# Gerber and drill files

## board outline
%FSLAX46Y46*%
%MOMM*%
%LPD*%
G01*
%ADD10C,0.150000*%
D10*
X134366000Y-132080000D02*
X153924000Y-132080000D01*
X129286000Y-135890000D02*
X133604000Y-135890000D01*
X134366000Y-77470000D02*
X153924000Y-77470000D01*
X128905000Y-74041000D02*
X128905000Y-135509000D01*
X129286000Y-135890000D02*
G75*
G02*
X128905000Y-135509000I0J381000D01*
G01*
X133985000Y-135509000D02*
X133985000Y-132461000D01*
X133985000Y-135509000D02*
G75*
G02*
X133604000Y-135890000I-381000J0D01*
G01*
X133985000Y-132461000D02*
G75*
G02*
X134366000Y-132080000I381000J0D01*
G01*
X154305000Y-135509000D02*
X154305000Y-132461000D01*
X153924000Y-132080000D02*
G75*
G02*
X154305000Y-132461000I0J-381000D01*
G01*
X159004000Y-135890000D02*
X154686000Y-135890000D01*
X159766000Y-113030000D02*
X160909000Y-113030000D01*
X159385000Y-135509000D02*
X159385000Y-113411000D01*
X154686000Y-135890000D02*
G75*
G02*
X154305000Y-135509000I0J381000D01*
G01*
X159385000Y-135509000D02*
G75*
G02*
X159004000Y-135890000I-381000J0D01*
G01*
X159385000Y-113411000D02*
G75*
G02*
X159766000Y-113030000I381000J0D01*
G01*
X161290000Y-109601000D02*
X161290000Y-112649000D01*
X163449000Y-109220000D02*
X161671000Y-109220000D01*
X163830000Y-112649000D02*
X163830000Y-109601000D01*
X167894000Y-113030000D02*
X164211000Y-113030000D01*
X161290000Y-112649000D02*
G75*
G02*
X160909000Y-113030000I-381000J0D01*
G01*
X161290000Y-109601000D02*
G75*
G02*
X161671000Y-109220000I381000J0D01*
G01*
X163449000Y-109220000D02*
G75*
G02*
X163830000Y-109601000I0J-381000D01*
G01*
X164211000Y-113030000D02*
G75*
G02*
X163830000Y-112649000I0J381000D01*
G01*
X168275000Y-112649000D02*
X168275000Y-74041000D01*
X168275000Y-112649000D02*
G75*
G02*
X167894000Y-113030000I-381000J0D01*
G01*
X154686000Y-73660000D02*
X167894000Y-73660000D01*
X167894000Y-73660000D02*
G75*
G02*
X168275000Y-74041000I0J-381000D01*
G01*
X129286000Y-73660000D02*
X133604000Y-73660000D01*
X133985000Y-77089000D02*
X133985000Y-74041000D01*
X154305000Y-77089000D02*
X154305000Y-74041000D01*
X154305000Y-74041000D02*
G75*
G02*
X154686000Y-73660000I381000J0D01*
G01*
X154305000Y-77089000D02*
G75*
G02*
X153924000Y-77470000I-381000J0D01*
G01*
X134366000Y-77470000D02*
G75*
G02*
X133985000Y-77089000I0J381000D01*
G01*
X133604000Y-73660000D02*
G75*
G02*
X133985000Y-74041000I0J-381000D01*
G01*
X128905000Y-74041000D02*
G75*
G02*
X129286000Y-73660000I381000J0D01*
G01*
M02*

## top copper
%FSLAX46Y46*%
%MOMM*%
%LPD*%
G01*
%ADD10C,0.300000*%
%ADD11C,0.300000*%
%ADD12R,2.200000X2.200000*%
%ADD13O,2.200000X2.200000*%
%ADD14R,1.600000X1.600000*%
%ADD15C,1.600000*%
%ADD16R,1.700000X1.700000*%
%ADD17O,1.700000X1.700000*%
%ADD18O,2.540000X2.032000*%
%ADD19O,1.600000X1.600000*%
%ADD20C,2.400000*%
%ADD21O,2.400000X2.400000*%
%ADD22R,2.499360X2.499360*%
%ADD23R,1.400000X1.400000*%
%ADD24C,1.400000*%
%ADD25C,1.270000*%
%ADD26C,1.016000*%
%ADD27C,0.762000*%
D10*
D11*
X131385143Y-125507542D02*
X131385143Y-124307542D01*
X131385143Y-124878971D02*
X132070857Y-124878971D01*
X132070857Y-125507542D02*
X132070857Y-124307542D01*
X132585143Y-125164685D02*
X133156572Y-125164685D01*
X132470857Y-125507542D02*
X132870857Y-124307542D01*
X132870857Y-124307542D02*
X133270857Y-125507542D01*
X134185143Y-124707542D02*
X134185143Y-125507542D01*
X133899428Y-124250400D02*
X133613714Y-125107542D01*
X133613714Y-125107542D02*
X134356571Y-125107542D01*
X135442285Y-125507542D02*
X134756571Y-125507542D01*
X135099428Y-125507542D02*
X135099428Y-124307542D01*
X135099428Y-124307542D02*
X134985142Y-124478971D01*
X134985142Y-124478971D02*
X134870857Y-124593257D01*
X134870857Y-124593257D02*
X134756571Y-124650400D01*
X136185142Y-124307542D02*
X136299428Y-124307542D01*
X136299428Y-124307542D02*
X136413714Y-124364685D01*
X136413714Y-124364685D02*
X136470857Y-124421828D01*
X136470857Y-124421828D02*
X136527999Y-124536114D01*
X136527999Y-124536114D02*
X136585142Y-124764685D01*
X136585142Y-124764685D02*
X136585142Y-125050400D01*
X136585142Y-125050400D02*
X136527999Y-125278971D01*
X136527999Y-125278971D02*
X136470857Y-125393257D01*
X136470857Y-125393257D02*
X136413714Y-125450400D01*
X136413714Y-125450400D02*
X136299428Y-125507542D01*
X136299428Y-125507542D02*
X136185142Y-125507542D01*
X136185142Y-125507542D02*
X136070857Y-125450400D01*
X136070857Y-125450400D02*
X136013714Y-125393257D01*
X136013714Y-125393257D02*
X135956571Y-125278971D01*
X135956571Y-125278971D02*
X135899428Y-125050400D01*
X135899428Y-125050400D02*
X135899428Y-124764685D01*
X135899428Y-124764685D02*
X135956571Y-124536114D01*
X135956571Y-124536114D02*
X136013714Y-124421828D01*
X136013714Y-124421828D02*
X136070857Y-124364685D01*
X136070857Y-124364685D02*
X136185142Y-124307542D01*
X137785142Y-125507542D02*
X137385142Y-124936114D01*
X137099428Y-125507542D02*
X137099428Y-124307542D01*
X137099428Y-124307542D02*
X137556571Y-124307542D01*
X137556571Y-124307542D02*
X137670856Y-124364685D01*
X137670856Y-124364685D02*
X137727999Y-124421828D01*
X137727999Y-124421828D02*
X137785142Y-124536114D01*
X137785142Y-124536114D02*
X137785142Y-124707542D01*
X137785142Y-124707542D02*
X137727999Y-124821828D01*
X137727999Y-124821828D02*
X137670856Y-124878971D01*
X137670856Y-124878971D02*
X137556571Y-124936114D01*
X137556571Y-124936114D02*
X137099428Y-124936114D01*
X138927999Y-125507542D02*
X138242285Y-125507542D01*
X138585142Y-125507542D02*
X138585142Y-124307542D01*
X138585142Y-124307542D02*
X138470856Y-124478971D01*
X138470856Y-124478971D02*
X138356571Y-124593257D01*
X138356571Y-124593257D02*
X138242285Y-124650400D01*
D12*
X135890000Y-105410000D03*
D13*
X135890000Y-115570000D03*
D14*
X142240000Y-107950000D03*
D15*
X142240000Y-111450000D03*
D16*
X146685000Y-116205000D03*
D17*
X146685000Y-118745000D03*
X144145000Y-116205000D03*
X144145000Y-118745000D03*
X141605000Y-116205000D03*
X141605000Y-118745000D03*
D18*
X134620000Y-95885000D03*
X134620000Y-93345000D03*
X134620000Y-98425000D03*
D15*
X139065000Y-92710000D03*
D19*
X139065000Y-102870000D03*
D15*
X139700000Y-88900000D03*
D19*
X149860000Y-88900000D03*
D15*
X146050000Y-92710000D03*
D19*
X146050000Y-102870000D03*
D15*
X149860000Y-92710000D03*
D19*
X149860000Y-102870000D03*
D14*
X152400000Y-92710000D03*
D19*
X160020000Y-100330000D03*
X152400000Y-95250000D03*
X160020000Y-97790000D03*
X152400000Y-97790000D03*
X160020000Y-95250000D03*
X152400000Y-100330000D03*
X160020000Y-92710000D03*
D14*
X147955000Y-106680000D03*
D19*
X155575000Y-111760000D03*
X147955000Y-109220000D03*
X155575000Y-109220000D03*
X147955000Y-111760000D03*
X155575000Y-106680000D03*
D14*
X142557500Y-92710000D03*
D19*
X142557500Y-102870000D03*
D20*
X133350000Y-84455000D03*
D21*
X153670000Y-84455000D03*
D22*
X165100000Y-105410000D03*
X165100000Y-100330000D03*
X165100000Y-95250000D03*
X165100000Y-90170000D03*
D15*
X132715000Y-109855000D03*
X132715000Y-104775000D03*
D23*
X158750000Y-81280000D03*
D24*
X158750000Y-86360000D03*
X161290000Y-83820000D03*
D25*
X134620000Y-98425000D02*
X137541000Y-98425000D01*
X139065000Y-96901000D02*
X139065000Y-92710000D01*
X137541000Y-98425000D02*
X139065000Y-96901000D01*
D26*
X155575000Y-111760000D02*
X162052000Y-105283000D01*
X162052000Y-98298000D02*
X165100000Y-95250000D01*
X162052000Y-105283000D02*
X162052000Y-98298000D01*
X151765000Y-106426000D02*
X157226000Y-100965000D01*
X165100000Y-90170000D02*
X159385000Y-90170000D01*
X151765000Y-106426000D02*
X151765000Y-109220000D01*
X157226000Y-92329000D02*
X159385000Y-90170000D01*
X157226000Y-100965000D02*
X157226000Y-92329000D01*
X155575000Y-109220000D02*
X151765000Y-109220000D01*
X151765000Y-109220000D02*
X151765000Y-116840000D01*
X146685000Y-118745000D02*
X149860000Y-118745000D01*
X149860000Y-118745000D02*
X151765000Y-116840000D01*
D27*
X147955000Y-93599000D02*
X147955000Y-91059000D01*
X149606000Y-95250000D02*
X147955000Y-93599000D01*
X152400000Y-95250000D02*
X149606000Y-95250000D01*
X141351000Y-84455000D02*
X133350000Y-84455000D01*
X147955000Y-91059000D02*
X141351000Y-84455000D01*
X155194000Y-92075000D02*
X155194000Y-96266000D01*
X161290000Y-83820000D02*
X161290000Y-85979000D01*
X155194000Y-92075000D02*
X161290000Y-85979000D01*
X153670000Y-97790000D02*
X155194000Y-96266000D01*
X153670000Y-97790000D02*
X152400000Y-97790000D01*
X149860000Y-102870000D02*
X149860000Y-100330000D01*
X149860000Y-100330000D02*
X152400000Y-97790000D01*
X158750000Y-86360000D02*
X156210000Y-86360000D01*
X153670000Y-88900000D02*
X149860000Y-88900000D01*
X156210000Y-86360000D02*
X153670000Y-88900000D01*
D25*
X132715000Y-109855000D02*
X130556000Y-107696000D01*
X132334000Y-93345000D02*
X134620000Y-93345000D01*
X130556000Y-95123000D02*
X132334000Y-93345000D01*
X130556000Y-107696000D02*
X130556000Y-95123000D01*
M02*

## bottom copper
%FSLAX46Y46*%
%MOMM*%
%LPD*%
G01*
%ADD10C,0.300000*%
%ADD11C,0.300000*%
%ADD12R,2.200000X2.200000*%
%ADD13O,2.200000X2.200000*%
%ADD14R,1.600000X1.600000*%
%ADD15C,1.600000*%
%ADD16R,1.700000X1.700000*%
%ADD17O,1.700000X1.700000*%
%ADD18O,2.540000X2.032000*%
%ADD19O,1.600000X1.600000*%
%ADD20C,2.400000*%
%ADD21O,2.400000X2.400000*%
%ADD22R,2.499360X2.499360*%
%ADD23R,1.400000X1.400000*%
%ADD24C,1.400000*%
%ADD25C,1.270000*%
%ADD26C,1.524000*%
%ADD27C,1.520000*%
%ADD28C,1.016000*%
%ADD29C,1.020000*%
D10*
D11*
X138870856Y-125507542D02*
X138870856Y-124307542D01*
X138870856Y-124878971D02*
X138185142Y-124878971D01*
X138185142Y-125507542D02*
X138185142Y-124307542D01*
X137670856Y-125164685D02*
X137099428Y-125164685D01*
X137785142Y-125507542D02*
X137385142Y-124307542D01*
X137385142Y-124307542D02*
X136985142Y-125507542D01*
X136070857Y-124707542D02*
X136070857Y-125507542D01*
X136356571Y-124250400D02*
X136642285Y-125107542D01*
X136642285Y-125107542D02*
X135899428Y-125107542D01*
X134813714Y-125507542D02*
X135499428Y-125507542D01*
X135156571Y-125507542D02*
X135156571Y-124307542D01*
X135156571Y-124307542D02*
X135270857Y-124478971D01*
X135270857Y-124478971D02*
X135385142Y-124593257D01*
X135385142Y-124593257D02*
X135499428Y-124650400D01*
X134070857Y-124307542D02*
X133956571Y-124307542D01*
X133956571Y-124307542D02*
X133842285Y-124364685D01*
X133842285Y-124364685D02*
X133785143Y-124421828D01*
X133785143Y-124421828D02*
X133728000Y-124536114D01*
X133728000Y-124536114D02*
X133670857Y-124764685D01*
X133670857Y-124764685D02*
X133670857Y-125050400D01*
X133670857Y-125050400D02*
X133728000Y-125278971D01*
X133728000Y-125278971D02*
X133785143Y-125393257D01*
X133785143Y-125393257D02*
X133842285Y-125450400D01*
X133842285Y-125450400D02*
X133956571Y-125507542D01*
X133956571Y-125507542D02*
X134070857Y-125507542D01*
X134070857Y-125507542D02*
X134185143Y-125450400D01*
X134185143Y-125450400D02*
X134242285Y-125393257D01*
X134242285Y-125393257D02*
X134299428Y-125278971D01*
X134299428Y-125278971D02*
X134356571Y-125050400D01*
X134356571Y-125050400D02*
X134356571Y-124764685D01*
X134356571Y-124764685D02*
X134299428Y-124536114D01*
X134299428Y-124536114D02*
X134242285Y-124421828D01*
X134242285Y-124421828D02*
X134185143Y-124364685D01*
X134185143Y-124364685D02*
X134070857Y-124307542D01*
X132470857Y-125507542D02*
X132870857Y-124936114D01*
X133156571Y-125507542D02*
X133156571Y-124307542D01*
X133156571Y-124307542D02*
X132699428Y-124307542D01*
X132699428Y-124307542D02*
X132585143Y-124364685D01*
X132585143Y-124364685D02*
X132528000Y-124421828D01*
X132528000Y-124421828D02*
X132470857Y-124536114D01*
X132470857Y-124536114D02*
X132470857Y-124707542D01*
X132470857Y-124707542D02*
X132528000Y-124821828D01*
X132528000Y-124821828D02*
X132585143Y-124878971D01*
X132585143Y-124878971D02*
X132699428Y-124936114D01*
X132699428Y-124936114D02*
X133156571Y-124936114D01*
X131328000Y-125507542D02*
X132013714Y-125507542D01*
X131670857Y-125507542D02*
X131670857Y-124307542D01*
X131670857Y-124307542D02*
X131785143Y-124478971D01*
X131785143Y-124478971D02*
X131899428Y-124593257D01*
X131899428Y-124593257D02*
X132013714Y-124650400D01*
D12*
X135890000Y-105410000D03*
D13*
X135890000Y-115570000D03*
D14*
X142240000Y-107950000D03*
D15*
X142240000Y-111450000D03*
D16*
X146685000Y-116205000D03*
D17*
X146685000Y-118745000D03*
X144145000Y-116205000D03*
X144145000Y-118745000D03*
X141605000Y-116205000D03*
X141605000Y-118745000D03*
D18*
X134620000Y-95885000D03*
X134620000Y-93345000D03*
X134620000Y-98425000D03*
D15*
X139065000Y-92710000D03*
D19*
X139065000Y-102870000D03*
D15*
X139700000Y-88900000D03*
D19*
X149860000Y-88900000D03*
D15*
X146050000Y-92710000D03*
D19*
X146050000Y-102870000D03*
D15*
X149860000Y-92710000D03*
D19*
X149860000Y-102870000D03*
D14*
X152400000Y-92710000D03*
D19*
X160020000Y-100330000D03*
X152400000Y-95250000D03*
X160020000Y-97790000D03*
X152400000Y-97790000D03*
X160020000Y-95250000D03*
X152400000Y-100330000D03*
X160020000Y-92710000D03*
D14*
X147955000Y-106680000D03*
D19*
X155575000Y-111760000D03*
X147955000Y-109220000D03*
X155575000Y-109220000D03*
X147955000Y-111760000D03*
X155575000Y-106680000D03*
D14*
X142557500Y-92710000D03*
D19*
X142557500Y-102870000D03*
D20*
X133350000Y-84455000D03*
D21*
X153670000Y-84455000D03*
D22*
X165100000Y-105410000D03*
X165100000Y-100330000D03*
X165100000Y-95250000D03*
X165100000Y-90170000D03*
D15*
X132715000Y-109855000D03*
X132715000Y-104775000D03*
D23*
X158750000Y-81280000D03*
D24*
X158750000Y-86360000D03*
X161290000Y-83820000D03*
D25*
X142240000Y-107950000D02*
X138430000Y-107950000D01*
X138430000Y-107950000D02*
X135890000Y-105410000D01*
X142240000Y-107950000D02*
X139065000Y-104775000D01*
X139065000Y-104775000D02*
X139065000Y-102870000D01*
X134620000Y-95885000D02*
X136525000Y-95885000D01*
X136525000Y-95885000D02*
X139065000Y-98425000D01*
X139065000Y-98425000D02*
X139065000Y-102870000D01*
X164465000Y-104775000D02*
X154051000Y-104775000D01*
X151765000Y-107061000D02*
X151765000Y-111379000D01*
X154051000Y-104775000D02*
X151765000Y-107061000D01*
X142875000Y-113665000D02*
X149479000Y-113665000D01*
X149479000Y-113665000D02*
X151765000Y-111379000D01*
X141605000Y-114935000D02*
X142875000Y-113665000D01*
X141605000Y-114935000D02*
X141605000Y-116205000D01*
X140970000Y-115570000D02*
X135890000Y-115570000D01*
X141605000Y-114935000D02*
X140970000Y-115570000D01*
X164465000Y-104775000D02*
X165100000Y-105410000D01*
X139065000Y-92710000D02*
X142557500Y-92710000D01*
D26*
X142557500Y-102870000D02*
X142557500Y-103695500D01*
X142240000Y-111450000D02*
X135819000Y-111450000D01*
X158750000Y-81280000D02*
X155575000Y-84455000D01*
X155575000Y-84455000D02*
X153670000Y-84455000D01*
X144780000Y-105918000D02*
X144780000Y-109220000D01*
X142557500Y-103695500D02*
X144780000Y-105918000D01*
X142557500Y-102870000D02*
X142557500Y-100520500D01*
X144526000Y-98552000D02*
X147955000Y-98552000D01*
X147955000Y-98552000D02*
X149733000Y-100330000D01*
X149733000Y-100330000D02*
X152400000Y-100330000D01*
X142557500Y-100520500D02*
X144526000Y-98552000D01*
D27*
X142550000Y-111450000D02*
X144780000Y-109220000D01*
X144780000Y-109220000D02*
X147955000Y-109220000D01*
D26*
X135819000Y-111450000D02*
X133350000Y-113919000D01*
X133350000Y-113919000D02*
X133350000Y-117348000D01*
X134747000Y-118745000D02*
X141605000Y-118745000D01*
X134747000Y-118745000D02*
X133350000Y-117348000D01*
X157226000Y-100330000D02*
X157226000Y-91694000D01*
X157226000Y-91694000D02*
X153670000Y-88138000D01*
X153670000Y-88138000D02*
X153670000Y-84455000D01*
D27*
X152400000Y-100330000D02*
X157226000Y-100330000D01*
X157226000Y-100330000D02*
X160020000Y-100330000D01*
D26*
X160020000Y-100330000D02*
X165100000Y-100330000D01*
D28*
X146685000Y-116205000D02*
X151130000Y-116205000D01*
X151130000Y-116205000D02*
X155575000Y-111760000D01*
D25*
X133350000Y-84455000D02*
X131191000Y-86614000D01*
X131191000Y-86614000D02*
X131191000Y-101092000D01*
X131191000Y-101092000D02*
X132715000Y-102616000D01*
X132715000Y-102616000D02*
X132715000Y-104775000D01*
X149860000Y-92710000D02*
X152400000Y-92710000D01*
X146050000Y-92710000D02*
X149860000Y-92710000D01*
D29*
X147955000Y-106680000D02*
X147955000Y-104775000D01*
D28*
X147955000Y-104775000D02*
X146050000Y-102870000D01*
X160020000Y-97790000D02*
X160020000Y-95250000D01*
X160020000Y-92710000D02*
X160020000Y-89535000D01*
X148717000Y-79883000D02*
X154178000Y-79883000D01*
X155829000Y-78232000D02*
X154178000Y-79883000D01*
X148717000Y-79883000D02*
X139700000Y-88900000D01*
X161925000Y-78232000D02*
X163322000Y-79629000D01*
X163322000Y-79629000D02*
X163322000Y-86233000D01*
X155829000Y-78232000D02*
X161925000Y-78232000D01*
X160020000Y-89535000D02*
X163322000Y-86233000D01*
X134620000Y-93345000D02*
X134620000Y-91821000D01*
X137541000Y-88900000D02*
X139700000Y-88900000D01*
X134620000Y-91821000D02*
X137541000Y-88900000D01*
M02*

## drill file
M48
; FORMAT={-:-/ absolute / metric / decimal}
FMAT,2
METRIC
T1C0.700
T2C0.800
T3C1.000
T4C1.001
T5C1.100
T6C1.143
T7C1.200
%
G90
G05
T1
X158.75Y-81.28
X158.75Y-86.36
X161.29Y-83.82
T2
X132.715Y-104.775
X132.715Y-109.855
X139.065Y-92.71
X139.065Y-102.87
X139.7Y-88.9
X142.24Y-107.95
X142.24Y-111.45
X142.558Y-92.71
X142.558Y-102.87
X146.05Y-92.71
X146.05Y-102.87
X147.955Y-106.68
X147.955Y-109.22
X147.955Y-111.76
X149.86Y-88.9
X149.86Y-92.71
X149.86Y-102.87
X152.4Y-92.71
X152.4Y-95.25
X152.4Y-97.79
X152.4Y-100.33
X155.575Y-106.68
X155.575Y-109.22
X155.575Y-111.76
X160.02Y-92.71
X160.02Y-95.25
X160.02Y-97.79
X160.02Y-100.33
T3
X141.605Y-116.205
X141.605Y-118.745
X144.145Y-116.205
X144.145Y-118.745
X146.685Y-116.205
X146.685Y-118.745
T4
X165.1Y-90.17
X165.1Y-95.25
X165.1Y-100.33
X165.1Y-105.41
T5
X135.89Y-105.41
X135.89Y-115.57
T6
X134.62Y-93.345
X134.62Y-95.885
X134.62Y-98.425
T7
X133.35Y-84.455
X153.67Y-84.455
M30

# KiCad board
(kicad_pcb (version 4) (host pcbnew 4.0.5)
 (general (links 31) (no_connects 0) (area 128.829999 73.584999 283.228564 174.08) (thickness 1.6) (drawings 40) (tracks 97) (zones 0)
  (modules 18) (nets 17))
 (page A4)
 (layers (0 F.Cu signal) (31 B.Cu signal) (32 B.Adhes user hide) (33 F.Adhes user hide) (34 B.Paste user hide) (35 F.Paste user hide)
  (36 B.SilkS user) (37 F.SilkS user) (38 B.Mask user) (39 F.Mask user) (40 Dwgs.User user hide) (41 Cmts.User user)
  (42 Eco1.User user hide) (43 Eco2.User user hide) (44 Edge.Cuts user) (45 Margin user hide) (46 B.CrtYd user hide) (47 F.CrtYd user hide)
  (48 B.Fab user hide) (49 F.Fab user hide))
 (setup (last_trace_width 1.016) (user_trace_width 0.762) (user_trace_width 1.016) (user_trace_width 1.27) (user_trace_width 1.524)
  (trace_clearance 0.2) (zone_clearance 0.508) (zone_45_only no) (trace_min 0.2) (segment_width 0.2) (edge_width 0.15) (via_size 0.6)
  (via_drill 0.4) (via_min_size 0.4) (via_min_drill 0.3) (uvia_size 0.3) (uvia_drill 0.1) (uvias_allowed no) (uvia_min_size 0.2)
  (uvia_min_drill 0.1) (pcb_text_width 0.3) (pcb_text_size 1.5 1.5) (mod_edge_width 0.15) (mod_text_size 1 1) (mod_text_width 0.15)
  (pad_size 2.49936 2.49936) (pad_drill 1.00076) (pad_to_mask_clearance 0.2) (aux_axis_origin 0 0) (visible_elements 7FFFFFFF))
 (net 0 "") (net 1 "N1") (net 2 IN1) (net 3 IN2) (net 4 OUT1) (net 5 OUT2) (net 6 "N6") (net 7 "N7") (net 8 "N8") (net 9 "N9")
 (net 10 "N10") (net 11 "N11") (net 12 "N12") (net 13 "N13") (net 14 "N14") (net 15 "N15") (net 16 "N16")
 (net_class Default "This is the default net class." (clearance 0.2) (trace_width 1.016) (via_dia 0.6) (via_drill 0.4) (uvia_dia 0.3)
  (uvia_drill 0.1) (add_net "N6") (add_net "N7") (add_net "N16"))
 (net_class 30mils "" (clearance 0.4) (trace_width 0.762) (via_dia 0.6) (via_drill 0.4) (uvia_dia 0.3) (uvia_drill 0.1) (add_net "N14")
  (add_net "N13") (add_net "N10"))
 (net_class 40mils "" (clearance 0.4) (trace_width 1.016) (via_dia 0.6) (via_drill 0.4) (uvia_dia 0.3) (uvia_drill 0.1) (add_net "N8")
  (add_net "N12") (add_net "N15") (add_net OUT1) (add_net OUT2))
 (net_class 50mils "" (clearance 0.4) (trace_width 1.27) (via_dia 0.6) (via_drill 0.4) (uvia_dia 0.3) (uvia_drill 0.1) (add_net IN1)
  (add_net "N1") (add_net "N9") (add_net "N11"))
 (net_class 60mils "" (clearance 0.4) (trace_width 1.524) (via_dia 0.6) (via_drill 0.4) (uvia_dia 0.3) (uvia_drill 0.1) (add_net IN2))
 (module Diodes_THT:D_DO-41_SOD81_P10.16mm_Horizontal (layer F.Cu) (at 135.89 105.41 270)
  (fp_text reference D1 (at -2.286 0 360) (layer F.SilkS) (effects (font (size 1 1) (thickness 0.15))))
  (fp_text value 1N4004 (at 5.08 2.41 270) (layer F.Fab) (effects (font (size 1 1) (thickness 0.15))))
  (pad 1 thru_hole rect (at 0 0 270) (size 2.2 2.2) (drill 1.1) (layers *.Cu *.Mask) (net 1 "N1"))
  (pad 2 thru_hole oval (at 10.16 0 270) (size 2.2 2.2) (drill 1.1) (layers *.Cu *.Mask) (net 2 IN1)))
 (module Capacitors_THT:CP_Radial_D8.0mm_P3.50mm (layer F.Cu) (at 142.24 107.95 270)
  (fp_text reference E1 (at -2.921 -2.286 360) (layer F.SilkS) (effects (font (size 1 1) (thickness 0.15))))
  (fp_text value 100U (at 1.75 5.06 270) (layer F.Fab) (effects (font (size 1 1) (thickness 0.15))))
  (pad 1 thru_hole rect (at 0 0 270) (size 1.6 1.6) (drill 0.8) (layers *.Cu *.Mask) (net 1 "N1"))
  (pad 2 thru_hole circle (at 3.5 0 270) (size 1.6 1.6) (drill 0.8) (layers *.Cu *.Mask) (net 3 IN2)))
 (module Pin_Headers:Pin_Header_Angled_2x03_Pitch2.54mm (layer F.Cu) (at 146.685 116.205 270)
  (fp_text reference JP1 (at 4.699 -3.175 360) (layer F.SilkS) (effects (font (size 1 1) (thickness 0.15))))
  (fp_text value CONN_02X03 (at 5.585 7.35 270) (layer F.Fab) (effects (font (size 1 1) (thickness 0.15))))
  (pad 1 thru_hole rect (at 0 0 270) (size 1.7 1.7) (drill 1) (layers *.Cu *.Mask) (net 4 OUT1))
  (pad 2 thru_hole oval (at 2.54 0 270) (size 1.7 1.7) (drill 1) (layers *.Cu *.Mask) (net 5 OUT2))
  (pad 3 thru_hole oval (at 0 2.54 270) (size 1.7 1.7) (drill 1) (layers *.Cu *.Mask) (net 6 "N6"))
  (pad 4 thru_hole oval (at 2.54 2.54 270) (size 1.7 1.7) (drill 1) (layers *.Cu *.Mask) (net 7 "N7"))
  (pad 5 thru_hole oval (at 0 5.08 270) (size 1.7 1.7) (drill 1) (layers *.Cu *.Mask) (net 2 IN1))
  (pad 6 thru_hole oval (at 2.54 5.08 270) (size 1.7 1.7) (drill 1) (layers *.Cu *.Mask) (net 3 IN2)))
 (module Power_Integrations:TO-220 (layer F.Cu) (at 134.62 95.885 90)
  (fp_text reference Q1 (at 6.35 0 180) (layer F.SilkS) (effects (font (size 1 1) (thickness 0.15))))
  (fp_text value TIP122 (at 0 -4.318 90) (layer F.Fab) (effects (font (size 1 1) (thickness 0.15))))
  (pad 2 thru_hole oval (at 0 0 90) (size 2.032 2.54) (drill 1.143) (layers *.Cu *.Mask) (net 1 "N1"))
  (pad 3 thru_hole oval (at 2.54 0 90) (size 2.032 2.54) (drill 1.143) (layers *.Cu *.Mask) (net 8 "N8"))
  (pad 1 thru_hole oval (at -2.54 0 90) (size 2.032 2.54) (drill 1.143) (layers *.Cu *.Mask) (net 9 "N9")))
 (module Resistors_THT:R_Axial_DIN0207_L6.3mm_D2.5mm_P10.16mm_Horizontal (layer F.Cu) (at 139.065 92.71 270)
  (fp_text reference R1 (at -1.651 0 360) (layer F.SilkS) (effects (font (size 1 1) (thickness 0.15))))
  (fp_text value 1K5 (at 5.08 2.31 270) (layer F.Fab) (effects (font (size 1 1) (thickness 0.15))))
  (pad 1 thru_hole circle (at 0 0 270) (size 1.6 1.6) (drill 0.8) (layers *.Cu *.Mask) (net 9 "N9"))
  (pad 2 thru_hole oval (at 10.16 0 270) (size 1.6 1.6) (drill 0.8) (layers *.Cu *.Mask) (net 1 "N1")))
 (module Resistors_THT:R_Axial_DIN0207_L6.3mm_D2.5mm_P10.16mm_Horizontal (layer F.Cu) (at 139.7 88.9)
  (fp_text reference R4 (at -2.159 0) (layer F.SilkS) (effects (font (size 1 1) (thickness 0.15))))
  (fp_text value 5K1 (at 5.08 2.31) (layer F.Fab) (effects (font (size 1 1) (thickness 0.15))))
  (pad 1 thru_hole circle (at 0 0) (size 1.6 1.6) (drill 0.8) (layers *.Cu *.Mask) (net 8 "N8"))
  (pad 2 thru_hole oval (at 10.16 0) (size 1.6 1.6) (drill 0.8) (layers *.Cu *.Mask) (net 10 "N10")))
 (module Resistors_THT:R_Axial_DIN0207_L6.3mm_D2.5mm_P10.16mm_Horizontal (layer F.Cu) (at 146.05 92.71 270)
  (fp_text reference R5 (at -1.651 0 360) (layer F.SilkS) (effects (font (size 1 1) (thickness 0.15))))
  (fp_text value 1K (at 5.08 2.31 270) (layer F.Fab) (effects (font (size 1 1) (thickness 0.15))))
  (pad 1 thru_hole circle (at 0 0 270) (size 1.6 1.6) (drill 0.8) (layers *.Cu *.Mask) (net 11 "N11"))
  (pad 2 thru_hole oval (at 10.16 0 270) (size 1.6 1.6) (drill 0.8) (layers *.Cu *.Mask) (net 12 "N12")))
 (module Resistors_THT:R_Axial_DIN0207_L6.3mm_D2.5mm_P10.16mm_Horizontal (layer F.Cu) (at 149.86 92.71 270)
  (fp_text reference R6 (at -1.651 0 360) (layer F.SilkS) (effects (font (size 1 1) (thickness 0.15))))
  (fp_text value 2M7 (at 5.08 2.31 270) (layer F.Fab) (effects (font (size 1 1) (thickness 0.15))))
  (pad 1 thru_hole circle (at 0 0 270) (size 1.6 1.6) (drill 0.8) (layers *.Cu *.Mask) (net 11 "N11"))
  (pad 2 thru_hole oval (at 10.16 0 270) (size 1.6 1.6) (drill 0.8) (layers *.Cu *.Mask) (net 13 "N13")))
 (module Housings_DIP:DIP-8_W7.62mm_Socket (layer F.Cu) (at 152.4 92.71)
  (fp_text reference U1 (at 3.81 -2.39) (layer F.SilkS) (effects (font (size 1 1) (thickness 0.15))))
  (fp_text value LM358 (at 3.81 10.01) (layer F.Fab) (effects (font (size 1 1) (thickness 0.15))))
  (pad 1 thru_hole rect (at 0 0) (size 1.6 1.6) (drill 0.8) (layers *.Cu *.Mask) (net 11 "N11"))
  (pad 5 thru_hole oval (at 7.62 7.62) (size 1.6 1.6) (drill 0.8) (layers *.Cu *.Mask) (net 3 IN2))
  (pad 2 thru_hole oval (at 0 2.54) (size 1.6 1.6) (drill 0.8) (layers *.Cu *.Mask) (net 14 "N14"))
  (pad 6 thru_hole oval (at 7.62 5.08) (size 1.6 1.6) (drill 0.8) (layers *.Cu *.Mask) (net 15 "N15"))
  (pad 3 thru_hole oval (at 0 5.08) (size 1.6 1.6) (drill 0.8) (layers *.Cu *.Mask) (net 13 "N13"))
  (pad 7 thru_hole oval (at 7.62 2.54) (size 1.6 1.6) (drill 0.8) (layers *.Cu *.Mask) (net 15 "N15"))
  (pad 4 thru_hole oval (at 0 7.62) (size 1.6 1.6) (drill 0.8) (layers *.Cu *.Mask) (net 3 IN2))
  (pad 8 thru_hole oval (at 7.62 0) (size 1.6 1.6) (drill 0.8) (layers *.Cu *.Mask) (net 8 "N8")))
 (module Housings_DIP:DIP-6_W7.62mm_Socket (layer F.Cu) (at 147.955 106.68)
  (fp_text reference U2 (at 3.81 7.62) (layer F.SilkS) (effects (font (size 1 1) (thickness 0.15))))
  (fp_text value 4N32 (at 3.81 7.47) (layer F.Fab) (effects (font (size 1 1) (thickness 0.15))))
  (pad 1 thru_hole rect (at 0 0) (size 1.6 1.6) (drill 0.8) (layers *.Cu *.Mask) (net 12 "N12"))
  (pad 4 thru_hole oval (at 7.62 5.08) (size 1.6 1.6) (drill 0.8) (layers *.Cu *.Mask) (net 4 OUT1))
  (pad 2 thru_hole oval (at 0 2.54) (size 1.6 1.6) (drill 0.8) (layers *.Cu *.Mask) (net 3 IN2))
  (pad 5 thru_hole oval (at 7.62 2.54) (size 1.6 1.6) (drill 0.8) (layers *.Cu *.Mask) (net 5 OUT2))
  (pad 3 thru_hole oval (at 0 5.08) (size 1.6 1.6) (drill 0.8) (layers *.Cu *.Mask))
  (pad 6 thru_hole oval (at 7.62 0) (size 1.6 1.6) (drill 0.8) (layers *.Cu *.Mask) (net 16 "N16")))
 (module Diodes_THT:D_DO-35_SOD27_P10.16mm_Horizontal (layer F.Cu) (at 142.5575 92.71 270)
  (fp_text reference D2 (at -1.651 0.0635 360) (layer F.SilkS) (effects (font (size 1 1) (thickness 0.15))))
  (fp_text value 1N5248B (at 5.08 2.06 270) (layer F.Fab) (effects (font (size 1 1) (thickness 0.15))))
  (pad 1 thru_hole rect (at 0 0 270) (size 1.6 1.6) (drill 0.8) (layers *.Cu *.Mask) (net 9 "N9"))
  (pad 2 thru_hole oval (at 10.16 0 270) (size 1.6 1.6) (drill 0.8) (layers *.Cu *.Mask) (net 3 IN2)))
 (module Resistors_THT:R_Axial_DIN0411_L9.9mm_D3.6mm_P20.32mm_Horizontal (layer F.Cu) (at 133.35 84.455)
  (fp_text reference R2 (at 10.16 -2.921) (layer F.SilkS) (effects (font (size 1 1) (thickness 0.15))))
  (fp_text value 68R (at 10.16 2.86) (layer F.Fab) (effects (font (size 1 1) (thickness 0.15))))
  (pad 1 thru_hole circle (at 0 0) (size 2.4 2.4) (drill 1.2) (layers *.Cu *.Mask) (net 14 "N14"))
  (pad 2 thru_hole oval (at 20.32 0) (size 2.4 2.4) (drill 1.2) (layers *.Cu *.Mask) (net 3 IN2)))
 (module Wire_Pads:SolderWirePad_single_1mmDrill (layer F.Cu) (at 165.1 105.41)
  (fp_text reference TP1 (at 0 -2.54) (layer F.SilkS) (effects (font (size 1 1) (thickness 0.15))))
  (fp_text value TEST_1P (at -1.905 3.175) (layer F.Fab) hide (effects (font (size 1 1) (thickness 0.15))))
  (pad 1 thru_hole rect (at 0 0) (size 2.49936 2.49936) (drill 1.00076) (layers *.Cu *.Mask) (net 2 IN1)))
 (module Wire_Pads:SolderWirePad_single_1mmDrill (layer F.Cu) (at 165.1 100.33)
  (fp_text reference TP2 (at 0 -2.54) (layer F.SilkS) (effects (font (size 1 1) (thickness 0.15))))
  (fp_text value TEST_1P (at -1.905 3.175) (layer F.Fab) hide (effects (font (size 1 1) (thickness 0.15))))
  (pad 1 thru_hole rect (at 0 0) (size 2.49936 2.49936) (drill 1.00076) (layers *.Cu *.Mask) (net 3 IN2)))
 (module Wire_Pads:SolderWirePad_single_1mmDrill (layer F.Cu) (at 165.1 95.25)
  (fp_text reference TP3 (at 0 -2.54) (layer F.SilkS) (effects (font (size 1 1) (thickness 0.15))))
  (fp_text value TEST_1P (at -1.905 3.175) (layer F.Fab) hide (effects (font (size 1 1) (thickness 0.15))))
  (pad 1 thru_hole rect (at 0 0) (size 2.49936 2.49936) (drill 1.00076) (layers *.Cu *.Mask) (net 4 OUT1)))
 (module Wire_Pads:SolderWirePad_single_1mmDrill (layer F.Cu) (at 165.1 90.17)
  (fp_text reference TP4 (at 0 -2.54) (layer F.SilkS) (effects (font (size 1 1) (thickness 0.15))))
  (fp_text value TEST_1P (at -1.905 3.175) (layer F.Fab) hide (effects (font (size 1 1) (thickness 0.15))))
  (pad 1 thru_hole rect (at 0 0) (size 2.49936 2.49936) (drill 1.00076) (layers *.Cu *.Mask) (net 5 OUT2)))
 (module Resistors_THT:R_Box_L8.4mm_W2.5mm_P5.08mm (layer F.Cu) (at 132.715 109.855 90)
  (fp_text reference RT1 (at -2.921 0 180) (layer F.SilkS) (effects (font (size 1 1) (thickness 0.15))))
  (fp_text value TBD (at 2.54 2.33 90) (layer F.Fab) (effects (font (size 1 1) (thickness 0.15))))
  (pad 1 thru_hole circle (at 0 0 90) (size 1.6 1.6) (drill 0.8) (layers *.Cu *.Mask) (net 8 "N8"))
  (pad 2 thru_hole circle (at 5.08 0 90) (size 1.6 1.6) (drill 0.8) (layers *.Cu *.Mask) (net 14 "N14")))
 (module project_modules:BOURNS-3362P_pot (layer F.Cu) (at 158.75 83.82 270)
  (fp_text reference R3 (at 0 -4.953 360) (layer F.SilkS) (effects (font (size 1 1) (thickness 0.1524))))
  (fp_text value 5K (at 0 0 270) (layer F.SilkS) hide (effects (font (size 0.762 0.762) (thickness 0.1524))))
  (pad 1 thru_hole rect (at -2.54 0 270) (size 1.4 1.4) (drill 0.7) (layers *.Cu *.Mask F.SilkS) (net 3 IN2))
  (pad 3 thru_hole circle (at 2.54 0 270) (size 1.4 1.4) (drill 0.7) (layers *.Cu *.Mask F.SilkS) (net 10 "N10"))
  (pad 2 thru_hole circle (at 0 -2.54 270) (size 1.4 1.4) (drill 0.7) (layers *.Cu *.Mask F.SilkS) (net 13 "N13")))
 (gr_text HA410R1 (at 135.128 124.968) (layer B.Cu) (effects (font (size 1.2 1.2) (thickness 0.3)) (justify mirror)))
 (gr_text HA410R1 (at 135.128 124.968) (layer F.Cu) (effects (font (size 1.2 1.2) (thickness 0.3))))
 (gr_line (start 134.366 132.08) (end 153.924 132.08) (angle 90) (layer Edge.Cuts) (width 0.15))
 (gr_line (start 129.286 135.89) (end 133.604 135.89) (angle 90) (layer Edge.Cuts) (width 0.15))
 (gr_line (start 134.366 77.47) (end 153.924 77.47) (angle 90) (layer Edge.Cuts) (width 0.15))
 (gr_line (start 128.905 74.041) (end 128.905 135.509) (angle 90) (layer Edge.Cuts) (width 0.15))
 (gr_arc (start 129.286 135.509) (end 129.286 135.89) (angle 90) (layer Edge.Cuts) (width 0.15))
 (gr_line (start 133.985 135.509) (end 133.985 132.461) (angle 90) (layer Edge.Cuts) (width 0.15))
 (gr_arc (start 133.604 135.509) (end 133.604 135.89) (angle -90) (layer Edge.Cuts) (width 0.15))
 (gr_arc (start 134.366 132.461) (end 134.366 132.08) (angle -90) (layer Edge.Cuts) (width 0.15))
 (gr_line (start 154.305 135.509) (end 154.305 132.461) (angle 90) (layer Edge.Cuts) (width 0.15))
 (gr_arc (start 153.924 132.461) (end 153.924 132.08) (angle 90) (layer Edge.Cuts) (width 0.15))
 (gr_line (start 159.004 135.89) (end 154.686 135.89) (angle 90) (layer Edge.Cuts) (width 0.15))
 (gr_line (start 159.766 113.03) (end 160.909 113.03) (angle 90) (layer Edge.Cuts) (width 0.15))
 (gr_line (start 159.385 135.509) (end 159.385 113.411) (angle 90) (layer Edge.Cuts) (width 0.15))
 (gr_arc (start 154.686 135.509) (end 154.686 135.89) (angle 90) (layer Edge.Cuts) (width 0.15))
 (gr_arc (start 159.004 135.509) (end 159.004 135.89) (angle -90) (layer Edge.Cuts) (width 0.15))
 (gr_arc (start 159.766 113.411) (end 159.766 113.03) (angle -90) (layer Edge.Cuts) (width 0.15))
 (gr_line (start 161.29 109.601) (end 161.29 112.649) (angle 90) (layer Edge.Cuts) (width 0.15))
 (gr_line (start 163.449 109.22) (end 161.671 109.22) (angle 90) (layer Edge.Cuts) (width 0.15))
 (gr_line (start 163.83 112.649) (end 163.83 109.601) (angle 90) (layer Edge.Cuts) (width 0.15))
 (gr_line (start 167.894 113.03) (end 164.211 113.03) (angle 90) (layer Edge.Cuts) (width 0.15))
 (gr_arc (start 160.909 112.649) (end 160.909 113.03) (angle -90) (layer Edge.Cuts) (width 0.15))
 (gr_arc (start 161.671 109.601) (end 161.671 109.22) (angle -90) (layer Edge.Cuts) (width 0.15))
 (gr_arc (start 163.449 109.601) (end 163.449 109.22) (angle 90) (layer Edge.Cuts) (width 0.15))
 (gr_arc (start 164.211 112.649) (end 164.211 113.03) (angle 90) (layer Edge.Cuts) (width 0.15))
 (gr_line (start 168.275 112.649) (end 168.275 74.041) (angle 90) (layer Edge.Cuts) (width 0.15))
 (gr_arc (start 167.894 112.649) (end 167.894 113.03) (angle -90) (layer Edge.Cuts) (width 0.15))
 (gr_line (start 154.686 73.66) (end 167.894 73.66) (angle 90) (layer Edge.Cuts) (width 0.15))
 (gr_arc (start 167.894 74.041) (end 167.894 73.66) (angle 90) (layer Edge.Cuts) (width 0.15))
 (gr_line (start 129.286 73.66) (end 133.604 73.66) (angle 90) (layer Edge.Cuts) (width 0.15))
 (gr_line (start 133.985 77.089) (end 133.985 74.041) (angle 90) (layer Edge.Cuts) (width 0.15))
 (gr_line (start 154.305 77.089) (end 154.305 74.041) (angle 90) (layer Edge.Cuts) (width 0.15))
 (gr_arc (start 154.686 74.041) (end 154.686 73.66) (angle -90) (layer Edge.Cuts) (width 0.15))
 (gr_arc (start 153.924 77.089) (end 153.924 77.47) (angle -90) (layer Edge.Cuts) (width 0.15))
 (gr_arc (start 134.366 77.089) (end 134.366 77.47) (angle 90) (layer Edge.Cuts) (width 0.15))
 (gr_arc (start 133.604 74.041) (end 133.604 73.66) (angle 90) (layer Edge.Cuts) (width 0.15))
 (gr_arc (start 129.286 74.041) (end 129.286 73.66) (angle -90) (layer Edge.Cuts) (width 0.15))
 (segment (start 142.24 107.95) (end 138.43 107.95) (width 1.27) (layer B.Cu) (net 1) (status 10))
 (segment (start 138.43 107.95) (end 135.89 105.41) (width 1.27) (layer B.Cu) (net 1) (status 20))
 (segment (start 142.24 107.95) (end 139.065 104.775) (width 1.27) (layer B.Cu) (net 1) (status 10))
 (segment (start 139.065 104.775) (end 139.065 102.87) (width 1.27) (layer B.Cu) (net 1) (status 20))
 (segment (start 134.62 95.885) (end 136.525 95.885) (width 1.27) (layer B.Cu) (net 1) (status 10))
 (segment (start 136.525 95.885) (end 139.065 98.425) (width 1.27) (layer B.Cu) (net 1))
 (segment (start 139.065 98.425) (end 139.065 102.87) (width 1.27) (layer B.Cu) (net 1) (status 20))
 (segment (start 164.465 104.775) (end 154.051 104.775) (width 1.27) (layer B.Cu) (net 2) (status 10))
 (segment (start 151.765 107.061) (end 151.765 111.379) (width 1.27) (layer B.Cu) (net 2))
 (segment (start 154.051 104.775) (end 151.765 107.061) (width 1.27) (layer B.Cu) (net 2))
 (segment (start 142.875 113.665) (end 149.479 113.665) (width 1.27) (layer B.Cu) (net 2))
 (segment (start 149.479 113.665) (end 151.765 111.379) (width 1.27) (layer B.Cu) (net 2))
 (segment (start 141.605 114.935) (end 142.875 113.665) (width 1.27) (layer B.Cu) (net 2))
 (segment (start 141.605 114.935) (end 141.605 116.205) (width 1.27) (layer B.Cu) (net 2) (status 20))
 (segment (start 140.97 115.57) (end 135.89 115.57) (width 1.27) (layer B.Cu) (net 2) (status 20))
 (segment (start 141.605 114.935) (end 140.97 115.57) (width 1.27) (layer B.Cu) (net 2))
 (segment (start 164.465 104.775) (end 165.1 105.41) (width 1.27) (layer B.Cu) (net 2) (status 30))
 (segment (start 134.62 98.425) (end 137.541 98.425) (width 1.27) (layer F.Cu) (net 9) (status 10))
 (segment (start 139.065 96.901) (end 139.065 92.71) (width 1.27) (layer F.Cu) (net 9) (status 20))
 (segment (start 137.541 98.425) (end 139.065 96.901) (width 1.27) (layer F.Cu) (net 9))
 (segment (start 139.065 92.71) (end 142.5575 92.71) (width 1.27) (layer B.Cu) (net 9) (status 30))
 (segment (start 142.5575 102.87) (end 142.5575 103.6955) (width 1.524) (layer B.Cu) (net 3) (status 10))
 (segment (start 142.24 111.45) (end 135.819 111.45) (width 1.524) (layer B.Cu) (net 3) (status 10))
 (segment (start 158.75 81.28) (end 155.575 84.455) (width 1.524) (layer B.Cu) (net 3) (status 10))
 (segment (start 155.575 84.455) (end 153.67 84.455) (width 1.524) (layer B.Cu) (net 3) (status 20))
 (segment (start 144.78 105.918) (end 144.78 109.22) (width 1.524) (layer B.Cu) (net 3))
 (segment (start 142.5575 103.6955) (end 144.78 105.918) (width 1.524) (layer B.Cu) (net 3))
 (segment (start 142.5575 102.87) (end 142.5575 100.5205) (width 1.524) (layer B.Cu) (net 3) (status 10))
 (segment (start 144.526 98.552) (end 147.955 98.552) (width 1.524) (layer B.Cu) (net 3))
 (segment (start 147.955 98.552) (end 149.733 100.33) (width 1.524) (layer B.Cu) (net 3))
 (segment (start 149.733 100.33) (end 152.4 100.33) (width 1.524) (layer B.Cu) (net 3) (status 20))
 (segment (start 142.5575 100.5205) (end 144.526 98.552) (width 1.524) (layer B.Cu) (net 3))
 (segment (start 142.55 111.45) (end 144.78 109.22) (width 1.52) (layer B.Cu) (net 3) (status 10))
 (segment (start 144.78 109.22) (end 147.955 109.22) (width 1.52) (layer B.Cu) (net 3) (status 20))
 (segment (start 135.819 111.45) (end 133.35 113.919) (width 1.524) (layer B.Cu) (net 3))
 (segment (start 133.35 113.919) (end 133.35 117.348) (width 1.524) (layer B.Cu) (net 3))
 (segment (start 134.747 118.745) (end 141.605 118.745) (width 1.524) (layer B.Cu) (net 3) (status 20))
 (segment (start 134.747 118.745) (end 133.35 117.348) (width 1.524) (layer B.Cu) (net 3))
 (segment (start 157.226 100.33) (end 157.226 91.694) (width 1.524) (layer B.Cu) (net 3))
 (segment (start 157.226 91.694) (end 153.67 88.138) (width 1.524) (layer B.Cu) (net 3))
 (segment (start 153.67 88.138) (end 153.67 84.455) (width 1.524) (layer B.Cu) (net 3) (status 20))
 (segment (start 152.4 100.33) (end 157.226 100.33) (width 1.52) (layer B.Cu) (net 3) (status 10))
 (segment (start 157.226 100.33) (end 160.02 100.33) (width 1.52) (layer B.Cu) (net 3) (status 20))
 (segment (start 160.02 100.33) (end 165.1 100.33) (width 1.524) (layer B.Cu) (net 3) (status 30))
 (segment (start 155.575 111.76) (end 162.052 105.283) (width 1.016) (layer F.Cu) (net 4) (status 10))
 (segment (start 162.052 98.298) (end 165.1 95.25) (width 1.016) (layer F.Cu) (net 4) (status 20))
 (segment (start 162.052 105.283) (end 162.052 98.298) (width 1.016) (layer F.Cu) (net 4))
 (segment (start 146.685 116.205) (end 151.13 116.205) (width 1.016) (layer B.Cu) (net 4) (status 10))
 (segment (start 151.13 116.205) (end 155.575 111.76) (width 1.016) (layer B.Cu) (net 4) (status 20))
 (segment (start 151.765 106.426) (end 157.226 100.965) (width 1.016) (layer F.Cu) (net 5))
 (segment (start 165.1 90.17) (end 159.385 90.17) (width 1.016) (layer F.Cu) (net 5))
 (segment (start 151.765 106.426) (end 151.765 109.22) (width 1.016) (layer F.Cu) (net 5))
 (segment (start 157.226 92.329) (end 159.385 90.17) (width 1.016) (layer F.Cu) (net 5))
 (segment (start 157.226 100.965) (end 157.226 92.329) (width 1.016) (layer F.Cu) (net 5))
 (segment (start 155.575 109.22) (end 151.765 109.22) (width 1.016) (layer F.Cu) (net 5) (status 10))
 (segment (start 151.765 109.22) (end 151.765 116.84) (width 1.016) (layer F.Cu) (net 5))
 (segment (start 146.685 118.745) (end 149.86 118.745) (width 1.016) (layer F.Cu) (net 5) (status 10))
 (segment (start 149.86 118.745) (end 151.765 116.84) (width 1.016) (layer F.Cu) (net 5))
 (segment (start 147.955 93.599) (end 147.955 91.059) (width 0.762) (layer F.Cu) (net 14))
 (segment (start 149.606 95.25) (end 147.955 93.599) (width 0.762) (layer F.Cu) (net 14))
 (segment (start 152.4 95.25) (end 149.606 95.25) (width 0.762) (layer F.Cu) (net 14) (status 10))
 (segment (start 141.351 84.455) (end 133.35 84.455) (width 0.762) (layer F.Cu) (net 14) (status 20))
 (segment (start 147.955 91.059) (end 141.351 84.455) (width 0.762) (layer F.Cu) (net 14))
 (segment (start 133.35 84.455) (end 131.191 86.614) (width 1.27) (layer B.Cu) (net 14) (status 10))
 (segment (start 131.191 86.614) (end 131.191 101.092) (width 1.27) (layer B.Cu) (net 14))
 (segment (start 131.191 101.092) (end 132.715 102.616) (width 1.27) (layer B.Cu) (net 14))
 (segment (start 132.715 102.616) (end 132.715 104.775) (width 1.27) (layer B.Cu) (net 14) (status 20))
 (segment (start 155.194 92.075) (end 155.194 96.266) (width 0.762) (layer F.Cu) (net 13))
 (segment (start 161.29 83.82) (end 161.29 85.979) (width 0.762) (layer F.Cu) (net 13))
 (segment (start 155.194 92.075) (end 161.29 85.979) (width 0.762) (layer F.Cu) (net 13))
 (segment (start 153.67 97.79) (end 155.194 96.266) (width 0.762) (layer F.Cu) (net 13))
 (segment (start 153.67 97.79) (end 152.4 97.79) (width 0.762) (layer F.Cu) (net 13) (status 10))
 (segment (start 149.86 102.87) (end 149.86 100.33) (width 0.762) (layer F.Cu) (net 13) (status 10))
 (segment (start 149.86 100.33) (end 152.4 97.79) (width 0.762) (layer F.Cu) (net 13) (status 20))
 (segment (start 149.86 92.71) (end 152.4 92.71) (width 1.27) (layer B.Cu) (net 11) (status 30))
 (segment (start 146.05 92.71) (end 149.86 92.71) (width 1.27) (layer B.Cu) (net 11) (status 30))
 (segment (start 147.955 106.68) (end 147.955 104.775) (width 1.02) (layer B.Cu) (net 12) (status 10))
 (segment (start 147.955 104.775) (end 146.05 102.87) (width 1.016) (layer B.Cu) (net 12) (status 20))
 (segment (start 160.02 97.79) (end 160.02 95.25) (width 1.016) (layer B.Cu) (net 15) (status 30))
 (segment (start 158.75 86.36) (end 156.21 86.36) (width 0.762) (layer F.Cu) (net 10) (status 10))
 (segment (start 153.67 88.9) (end 149.86 88.9) (width 0.762) (layer F.Cu) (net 10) (status 20))
 (segment (start 156.21 86.36) (end 153.67 88.9) (width 0.762) (layer F.Cu) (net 10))
 (segment (start 160.02 92.71) (end 160.02 89.535) (width 1.016) (layer B.Cu) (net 8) (status 10))
 (segment (start 148.717 79.883) (end 154.178 79.883) (width 1.016) (layer B.Cu) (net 8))
 (segment (start 155.829 78.232) (end 154.178 79.883) (width 1.016) (layer B.Cu) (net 8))
 (segment (start 148.717 79.883) (end 139.7 88.9) (width 1.016) (layer B.Cu) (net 8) (status 20))
 (segment (start 161.925 78.232) (end 163.322 79.629) (width 1.016) (layer B.Cu) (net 8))
 (segment (start 163.322 79.629) (end 163.322 86.233) (width 1.016) (layer B.Cu) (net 8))
 (segment (start 155.829 78.232) (end 161.925 78.232) (width 1.016) (layer B.Cu) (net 8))
 (segment (start 160.02 89.535) (end 163.322 86.233) (width 1.016) (layer B.Cu) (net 8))
 (segment (start 134.62 93.345) (end 134.62 91.821) (width 1.016) (layer B.Cu) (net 8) (status 10))
 (segment (start 137.541 88.9) (end 139.7 88.9) (width 1.016) (layer B.Cu) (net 8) (status 20))
 (segment (start 134.62 91.821) (end 137.541 88.9) (width 1.016) (layer B.Cu) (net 8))
 (segment (start 132.715 109.855) (end 130.556 107.696) (width 1.27) (layer F.Cu) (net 8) (status 10))
 (segment (start 132.334 93.345) (end 134.62 93.345) (width 1.27) (layer F.Cu) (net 8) (status 20))
 (segment (start 130.556 95.123) (end 132.334 93.345) (width 1.27) (layer F.Cu) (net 8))
 (segment (start 130.556 107.696) (end 130.556 95.123) (width 1.27) (layer F.Cu) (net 8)))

